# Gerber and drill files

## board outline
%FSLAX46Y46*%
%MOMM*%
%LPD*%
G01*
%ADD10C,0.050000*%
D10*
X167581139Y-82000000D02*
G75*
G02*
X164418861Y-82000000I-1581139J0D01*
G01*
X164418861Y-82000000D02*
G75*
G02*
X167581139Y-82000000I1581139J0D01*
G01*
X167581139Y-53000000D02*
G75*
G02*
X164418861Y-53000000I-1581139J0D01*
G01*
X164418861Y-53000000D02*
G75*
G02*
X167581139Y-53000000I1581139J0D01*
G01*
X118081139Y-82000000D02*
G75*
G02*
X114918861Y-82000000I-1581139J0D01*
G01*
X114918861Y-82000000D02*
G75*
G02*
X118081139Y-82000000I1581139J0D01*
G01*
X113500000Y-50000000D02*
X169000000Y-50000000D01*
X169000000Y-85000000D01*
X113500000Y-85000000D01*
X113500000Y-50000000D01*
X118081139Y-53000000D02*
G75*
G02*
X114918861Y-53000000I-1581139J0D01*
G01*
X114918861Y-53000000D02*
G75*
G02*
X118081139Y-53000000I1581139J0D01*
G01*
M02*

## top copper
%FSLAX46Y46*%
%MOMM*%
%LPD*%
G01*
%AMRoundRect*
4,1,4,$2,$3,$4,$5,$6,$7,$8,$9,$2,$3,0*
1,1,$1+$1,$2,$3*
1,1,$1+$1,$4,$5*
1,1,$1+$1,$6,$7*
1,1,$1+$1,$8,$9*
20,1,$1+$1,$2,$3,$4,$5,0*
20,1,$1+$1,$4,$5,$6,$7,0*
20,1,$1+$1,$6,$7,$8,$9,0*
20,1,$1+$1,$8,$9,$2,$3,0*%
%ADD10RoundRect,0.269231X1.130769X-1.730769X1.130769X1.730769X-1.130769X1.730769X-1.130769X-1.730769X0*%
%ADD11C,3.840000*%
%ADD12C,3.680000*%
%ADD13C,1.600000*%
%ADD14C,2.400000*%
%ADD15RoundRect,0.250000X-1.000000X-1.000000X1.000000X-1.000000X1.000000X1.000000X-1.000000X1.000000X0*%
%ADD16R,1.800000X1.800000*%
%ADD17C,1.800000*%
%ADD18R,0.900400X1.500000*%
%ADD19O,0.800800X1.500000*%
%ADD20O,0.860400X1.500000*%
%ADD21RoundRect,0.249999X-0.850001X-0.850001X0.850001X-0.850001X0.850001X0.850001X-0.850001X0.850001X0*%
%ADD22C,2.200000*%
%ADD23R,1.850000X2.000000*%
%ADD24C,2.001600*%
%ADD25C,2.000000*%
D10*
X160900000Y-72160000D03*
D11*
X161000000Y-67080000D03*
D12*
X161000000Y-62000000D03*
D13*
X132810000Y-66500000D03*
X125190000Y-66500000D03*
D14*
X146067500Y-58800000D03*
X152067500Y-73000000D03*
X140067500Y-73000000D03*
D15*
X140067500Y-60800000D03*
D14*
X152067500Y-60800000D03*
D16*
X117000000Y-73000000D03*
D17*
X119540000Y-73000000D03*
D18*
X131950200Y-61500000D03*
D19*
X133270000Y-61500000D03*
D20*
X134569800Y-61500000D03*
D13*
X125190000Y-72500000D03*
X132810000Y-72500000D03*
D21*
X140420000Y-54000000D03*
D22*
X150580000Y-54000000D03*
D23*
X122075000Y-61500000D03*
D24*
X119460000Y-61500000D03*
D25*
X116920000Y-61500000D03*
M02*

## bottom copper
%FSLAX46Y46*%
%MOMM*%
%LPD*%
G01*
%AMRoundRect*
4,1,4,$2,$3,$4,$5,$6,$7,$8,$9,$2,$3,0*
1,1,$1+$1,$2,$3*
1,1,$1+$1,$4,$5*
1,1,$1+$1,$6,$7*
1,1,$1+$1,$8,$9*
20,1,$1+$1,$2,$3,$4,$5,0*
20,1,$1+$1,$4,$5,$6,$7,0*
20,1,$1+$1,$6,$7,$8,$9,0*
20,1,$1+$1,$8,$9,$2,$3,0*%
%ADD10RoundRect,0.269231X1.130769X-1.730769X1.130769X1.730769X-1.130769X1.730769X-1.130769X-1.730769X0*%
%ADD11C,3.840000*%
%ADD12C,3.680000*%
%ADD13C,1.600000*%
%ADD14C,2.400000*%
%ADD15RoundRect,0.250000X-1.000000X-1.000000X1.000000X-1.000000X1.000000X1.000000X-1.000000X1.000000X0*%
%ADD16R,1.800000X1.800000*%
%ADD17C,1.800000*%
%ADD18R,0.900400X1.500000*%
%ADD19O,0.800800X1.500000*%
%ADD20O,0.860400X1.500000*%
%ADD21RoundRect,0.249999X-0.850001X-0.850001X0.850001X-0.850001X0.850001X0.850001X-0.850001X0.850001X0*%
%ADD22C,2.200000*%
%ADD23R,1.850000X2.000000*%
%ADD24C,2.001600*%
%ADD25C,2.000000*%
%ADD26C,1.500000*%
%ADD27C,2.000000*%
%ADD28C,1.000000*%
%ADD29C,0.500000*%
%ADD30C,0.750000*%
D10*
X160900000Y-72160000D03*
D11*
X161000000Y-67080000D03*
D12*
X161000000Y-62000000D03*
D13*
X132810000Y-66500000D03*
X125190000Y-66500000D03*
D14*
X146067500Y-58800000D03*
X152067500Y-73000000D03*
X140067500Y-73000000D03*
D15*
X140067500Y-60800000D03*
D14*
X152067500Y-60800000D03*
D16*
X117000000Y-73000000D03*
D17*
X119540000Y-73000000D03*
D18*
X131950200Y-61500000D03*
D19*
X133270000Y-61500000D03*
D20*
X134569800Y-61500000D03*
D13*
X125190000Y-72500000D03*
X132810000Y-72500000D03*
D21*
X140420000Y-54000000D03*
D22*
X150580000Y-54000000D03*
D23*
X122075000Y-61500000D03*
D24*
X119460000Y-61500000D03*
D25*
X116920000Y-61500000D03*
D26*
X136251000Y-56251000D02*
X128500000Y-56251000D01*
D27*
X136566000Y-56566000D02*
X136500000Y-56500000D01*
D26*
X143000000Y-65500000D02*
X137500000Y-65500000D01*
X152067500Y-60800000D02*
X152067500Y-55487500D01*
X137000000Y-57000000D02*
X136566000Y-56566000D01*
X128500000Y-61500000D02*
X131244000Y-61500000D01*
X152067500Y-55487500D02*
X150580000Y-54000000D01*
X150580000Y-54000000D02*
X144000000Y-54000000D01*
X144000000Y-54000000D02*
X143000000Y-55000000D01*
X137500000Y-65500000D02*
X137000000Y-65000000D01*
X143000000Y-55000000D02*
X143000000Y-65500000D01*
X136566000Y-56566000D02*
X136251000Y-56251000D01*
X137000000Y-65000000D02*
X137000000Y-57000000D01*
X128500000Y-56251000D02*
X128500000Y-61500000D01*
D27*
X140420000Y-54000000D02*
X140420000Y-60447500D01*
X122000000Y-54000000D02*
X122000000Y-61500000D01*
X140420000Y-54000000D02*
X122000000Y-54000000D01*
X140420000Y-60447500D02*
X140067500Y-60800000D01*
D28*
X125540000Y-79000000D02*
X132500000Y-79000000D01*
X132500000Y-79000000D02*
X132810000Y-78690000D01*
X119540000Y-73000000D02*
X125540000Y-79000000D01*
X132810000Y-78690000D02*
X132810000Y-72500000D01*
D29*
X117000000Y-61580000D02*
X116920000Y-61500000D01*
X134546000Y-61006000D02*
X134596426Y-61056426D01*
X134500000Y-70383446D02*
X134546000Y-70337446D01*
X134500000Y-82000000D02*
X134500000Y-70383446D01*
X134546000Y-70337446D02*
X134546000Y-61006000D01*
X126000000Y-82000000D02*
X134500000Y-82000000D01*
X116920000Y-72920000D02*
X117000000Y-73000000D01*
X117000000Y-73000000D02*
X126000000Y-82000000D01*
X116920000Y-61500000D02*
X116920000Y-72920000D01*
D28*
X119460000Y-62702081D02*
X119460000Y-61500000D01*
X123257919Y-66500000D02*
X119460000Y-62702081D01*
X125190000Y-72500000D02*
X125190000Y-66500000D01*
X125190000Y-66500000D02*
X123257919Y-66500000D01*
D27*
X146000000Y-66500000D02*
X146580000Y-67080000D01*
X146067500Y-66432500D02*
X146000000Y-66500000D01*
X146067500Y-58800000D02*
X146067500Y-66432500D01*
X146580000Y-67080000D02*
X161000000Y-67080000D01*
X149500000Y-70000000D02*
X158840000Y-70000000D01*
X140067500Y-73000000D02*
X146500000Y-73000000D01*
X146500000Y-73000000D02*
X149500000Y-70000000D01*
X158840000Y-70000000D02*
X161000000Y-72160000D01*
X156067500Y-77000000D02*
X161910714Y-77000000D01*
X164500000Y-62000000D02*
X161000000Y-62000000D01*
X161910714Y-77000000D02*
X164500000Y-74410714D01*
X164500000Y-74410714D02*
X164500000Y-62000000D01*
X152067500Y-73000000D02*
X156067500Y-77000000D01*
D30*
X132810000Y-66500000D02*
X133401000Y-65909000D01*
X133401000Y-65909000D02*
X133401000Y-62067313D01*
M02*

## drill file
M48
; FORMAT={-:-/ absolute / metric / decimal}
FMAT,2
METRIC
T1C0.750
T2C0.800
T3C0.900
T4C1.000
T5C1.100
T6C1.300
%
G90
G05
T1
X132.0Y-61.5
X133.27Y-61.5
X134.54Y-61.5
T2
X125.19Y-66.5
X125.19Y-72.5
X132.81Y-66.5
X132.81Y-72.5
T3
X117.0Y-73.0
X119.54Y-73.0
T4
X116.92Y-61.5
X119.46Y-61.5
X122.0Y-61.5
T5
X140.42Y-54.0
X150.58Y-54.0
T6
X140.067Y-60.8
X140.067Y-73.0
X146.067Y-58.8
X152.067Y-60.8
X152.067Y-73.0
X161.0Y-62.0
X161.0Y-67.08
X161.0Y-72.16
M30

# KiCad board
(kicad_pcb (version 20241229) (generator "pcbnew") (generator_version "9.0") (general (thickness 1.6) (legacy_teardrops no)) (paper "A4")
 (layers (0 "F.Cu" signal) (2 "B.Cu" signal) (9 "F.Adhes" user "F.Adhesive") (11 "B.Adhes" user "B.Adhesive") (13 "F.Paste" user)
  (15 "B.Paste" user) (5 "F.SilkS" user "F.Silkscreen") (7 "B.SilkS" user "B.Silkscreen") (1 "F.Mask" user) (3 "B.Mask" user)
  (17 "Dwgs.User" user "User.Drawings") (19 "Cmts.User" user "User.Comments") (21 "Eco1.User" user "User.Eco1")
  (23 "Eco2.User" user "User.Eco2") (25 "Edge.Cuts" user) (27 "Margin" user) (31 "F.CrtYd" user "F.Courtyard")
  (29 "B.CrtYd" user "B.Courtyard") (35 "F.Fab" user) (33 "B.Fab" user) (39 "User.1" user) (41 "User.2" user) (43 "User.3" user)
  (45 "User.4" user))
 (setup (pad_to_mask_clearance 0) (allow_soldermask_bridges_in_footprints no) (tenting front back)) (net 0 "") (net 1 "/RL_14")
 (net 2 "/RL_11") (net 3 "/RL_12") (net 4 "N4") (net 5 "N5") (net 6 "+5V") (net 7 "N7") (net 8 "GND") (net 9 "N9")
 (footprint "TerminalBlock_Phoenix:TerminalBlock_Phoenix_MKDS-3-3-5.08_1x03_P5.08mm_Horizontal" (layer "F.Cu") (at 161 72.16 90)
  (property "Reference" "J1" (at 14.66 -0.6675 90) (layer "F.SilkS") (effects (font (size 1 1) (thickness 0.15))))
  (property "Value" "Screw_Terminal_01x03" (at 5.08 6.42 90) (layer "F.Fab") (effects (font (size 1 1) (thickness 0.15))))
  (pad "1" thru_hole roundrect (at 0 0 90) (size 4 2.8) (drill 1.3 (offset 0 -0.1)) (layers "*.Cu" "*.Mask") (remove_unused_layers no)
   (roundrect_rratio 0.096154) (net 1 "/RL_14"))
  (pad "2" thru_hole circle (at 5.08 0 90) (size 3.84 3.84) (drill 1.3) (layers "*.Cu" "*.Mask") (remove_unused_layers no) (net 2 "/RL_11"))
  (pad "3" thru_hole circle (at 10.16 0 90) (size 3.68 3.68) (drill 1.3) (layers "*.Cu" "*.Mask") (remove_unused_layers no) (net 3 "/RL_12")))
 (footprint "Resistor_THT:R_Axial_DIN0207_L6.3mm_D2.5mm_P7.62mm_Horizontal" (layer "F.Cu") (at 132.81 66.5 180)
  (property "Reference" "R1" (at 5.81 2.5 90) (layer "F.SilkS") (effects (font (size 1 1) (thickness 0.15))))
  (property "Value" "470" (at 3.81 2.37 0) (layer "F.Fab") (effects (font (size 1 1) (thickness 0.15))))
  (pad "1" thru_hole circle (at 0 0 180) (size 1.6 1.6) (drill 0.8) (layers "*.Cu" "*.Mask") (remove_unused_layers no) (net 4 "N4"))
  (pad "2" thru_hole circle (at 7.62 0 180) (size 1.6 1.6) (drill 0.8) (layers "*.Cu" "*.Mask") (remove_unused_layers no) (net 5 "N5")))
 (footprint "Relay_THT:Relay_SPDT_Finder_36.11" (layer "F.Cu") (at 140.0675 60.8)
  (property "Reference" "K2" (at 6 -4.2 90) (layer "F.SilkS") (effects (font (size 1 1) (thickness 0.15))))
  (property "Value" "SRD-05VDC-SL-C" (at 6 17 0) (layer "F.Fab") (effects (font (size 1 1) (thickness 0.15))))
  (pad "11" thru_hole circle (at 6 -2) (size 2.4 2.4) (drill 1.3) (layers "*.Cu" "*.Mask") (remove_unused_layers no) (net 2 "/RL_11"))
  (pad "12" thru_hole circle (at 12 12.2) (size 2.4 2.4) (drill 1.3) (layers "*.Cu" "*.Mask") (remove_unused_layers no) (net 3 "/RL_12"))
  (pad "14" thru_hole circle (at 0 12.2) (size 2.4 2.4) (drill 1.3) (layers "*.Cu" "*.Mask") (remove_unused_layers no) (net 1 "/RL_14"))
  (pad "A1" thru_hole roundrect (at 0 0) (size 2.5 2.5) (drill 1.3) (layers "*.Cu" "*.Mask") (remove_unused_layers no)
   (roundrect_rratio 0.1) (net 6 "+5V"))
  (pad "A2" thru_hole circle (at 12 0) (size 2.4 2.4) (drill 1.3) (layers "*.Cu" "*.Mask") (remove_unused_layers no) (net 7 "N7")))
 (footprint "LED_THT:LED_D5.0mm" (layer "F.Cu") (at 117 73)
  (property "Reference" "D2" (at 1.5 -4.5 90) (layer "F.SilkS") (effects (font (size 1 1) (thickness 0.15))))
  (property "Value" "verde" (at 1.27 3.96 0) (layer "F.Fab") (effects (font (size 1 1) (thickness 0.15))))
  (pad "1" thru_hole rect (at 0 0) (size 1.8 1.8) (drill 0.9) (layers "*.Cu" "*.Mask") (remove_unused_layers no) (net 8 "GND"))
  (pad "2" thru_hole circle (at 2.54 0) (size 1.8 1.8) (drill 0.9) (layers "*.Cu" "*.Mask") (remove_unused_layers no) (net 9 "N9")))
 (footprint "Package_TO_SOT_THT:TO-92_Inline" (layer "F.Cu") (at 132 61.5)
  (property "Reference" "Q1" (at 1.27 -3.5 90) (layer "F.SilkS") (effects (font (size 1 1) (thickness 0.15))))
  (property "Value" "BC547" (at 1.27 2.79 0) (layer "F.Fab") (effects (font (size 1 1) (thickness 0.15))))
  (pad "1" thru_hole rect (at 0 0) (size 0.9004 1.5) (drill 0.75 (offset -0.0498 0)) (layers "*.Cu" "*.Mask") (remove_unused_layers no)
   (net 7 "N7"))
  (pad "2" thru_hole oval (at 1.27 0) (size 0.8008 1.5) (drill 0.75) (layers "*.Cu" "*.Mask") (remove_unused_layers no) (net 4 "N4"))
  (pad "3" thru_hole oval (at 2.54 0) (size 0.8604 1.5) (drill 0.75 (offset 0.0298 0)) (layers "*.Cu" "*.Mask") (remove_unused_layers no)
   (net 8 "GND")))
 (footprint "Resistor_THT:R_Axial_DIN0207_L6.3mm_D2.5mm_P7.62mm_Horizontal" (layer "F.Cu") (at 125.19 72.5)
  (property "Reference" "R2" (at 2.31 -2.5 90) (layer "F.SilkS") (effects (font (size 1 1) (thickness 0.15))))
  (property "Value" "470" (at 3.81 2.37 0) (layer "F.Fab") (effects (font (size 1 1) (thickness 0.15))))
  (pad "1" thru_hole circle (at 0 0) (size 1.6 1.6) (drill 0.8) (layers "*.Cu" "*.Mask") (remove_unused_layers no) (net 5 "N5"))
  (pad "2" thru_hole circle (at 7.62 0) (size 1.6 1.6) (drill 0.8) (layers "*.Cu" "*.Mask") (remove_unused_layers no) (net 9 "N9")))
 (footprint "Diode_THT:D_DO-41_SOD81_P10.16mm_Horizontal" (layer "F.Cu") (at 140.42 54)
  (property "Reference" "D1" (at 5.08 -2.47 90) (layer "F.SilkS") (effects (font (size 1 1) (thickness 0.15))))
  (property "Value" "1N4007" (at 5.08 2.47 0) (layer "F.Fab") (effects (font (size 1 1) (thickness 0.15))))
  (pad "1" thru_hole roundrect (at 0 0) (size 2.2 2.2) (drill 1.1) (layers "*.Cu" "*.Mask") (remove_unused_layers no)
   (roundrect_rratio 0.113636) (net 6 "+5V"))
  (pad "2" thru_hole circle (at 10.16 0) (size 2.2 2.2) (drill 1.1) (layers "*.Cu" "*.Mask") (remove_unused_layers no) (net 7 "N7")))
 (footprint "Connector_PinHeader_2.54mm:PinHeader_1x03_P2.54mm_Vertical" (layer "F.Cu") (at 122 61.5 -90)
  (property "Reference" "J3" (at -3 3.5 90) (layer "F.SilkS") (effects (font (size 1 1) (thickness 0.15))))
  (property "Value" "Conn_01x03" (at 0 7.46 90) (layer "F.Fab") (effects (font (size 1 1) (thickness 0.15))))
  (pad "1" thru_hole rect (at 0 0 270) (size 2 1.85) (drill 1 (offset 0 -0.075)) (layers "*.Cu" "*.Mask") (remove_unused_layers no)
   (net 6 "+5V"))
  (pad "2" thru_hole circle (at 0 2.54 270) (size 2.0016 2.0016) (drill 1) (layers "*.Cu" "*.Mask") (remove_unused_layers no) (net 5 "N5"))
  (pad "3" thru_hole circle (at 0 5.08 270) (size 2 2) (drill 1) (layers "*.Cu" "*.Mask") (remove_unused_layers no) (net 8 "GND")))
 (gr_circle (center 166 82) (end 166.5 83.5) (stroke (width 0.05) (type default)) (fill no) (layer "Edge.Cuts"))
 (gr_circle (center 166 53) (end 166.5 54.5) (stroke (width 0.05) (type default)) (fill no) (layer "Edge.Cuts"))
 (gr_circle (center 116.5 82) (end 117 83.5) (stroke (width 0.05) (type default)) (fill no) (layer "Edge.Cuts"))
 (gr_rect (start 113.5 50) (end 169 85) (stroke (width 0.05) (type default)) (fill no) (layer "Edge.Cuts"))
 (gr_circle (center 116.5 53) (end 117 54.5) (stroke (width 0.05) (type default)) (fill no) (layer "Edge.Cuts"))
 (segment (start 136.251 56.251) (end 128.5 56.251) (width 1.5) (layer "B.Cu") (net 7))
 (segment (start 136.566 56.566) (end 136.5 56.5) (width 2) (layer "B.Cu") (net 7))
 (segment (start 143 65.5) (end 137.5 65.5) (width 1.5) (layer "B.Cu") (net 7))
 (segment (start 152.0675 60.8) (end 152.0675 55.4875) (width 1.5) (layer "B.Cu") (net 7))
 (segment (start 137 57) (end 136.566 56.566) (width 1.5) (layer "B.Cu") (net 7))
 (segment (start 128.5 61.5) (end 131.244 61.5) (width 1.5) (layer "B.Cu") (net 7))
 (segment (start 152.0675 55.4875) (end 150.58 54) (width 1.5) (layer "B.Cu") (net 7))
 (segment (start 150.58 54) (end 144 54) (width 1.5) (layer "B.Cu") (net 7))
 (segment (start 144 54) (end 143 55) (width 1.5) (layer "B.Cu") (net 7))
 (segment (start 137.5 65.5) (end 137 65) (width 1.5) (layer "B.Cu") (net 7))
 (segment (start 143 55) (end 143 65.5) (width 1.5) (layer "B.Cu") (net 7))
 (segment (start 136.566 56.566) (end 136.251 56.251) (width 1.5) (layer "B.Cu") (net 7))
 (segment (start 137 65) (end 137 57) (width 1.5) (layer "B.Cu") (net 7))
 (segment (start 128.5 56.251) (end 128.5 61.5) (width 1.5) (layer "B.Cu") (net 7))
 (segment (start 140.42 54) (end 140.42 60.4475) (width 2) (layer "B.Cu") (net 6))
 (segment (start 122 54) (end 122 61.5) (width 2) (layer "B.Cu") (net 6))
 (segment (start 140.42 54) (end 122 54) (width 2) (layer "B.Cu") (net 6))
 (segment (start 140.42 60.4475) (end 140.0675 60.8) (width 2) (layer "B.Cu") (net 6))
 (segment (start 125.54 79) (end 132.5 79) (width 1) (layer "B.Cu") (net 9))
 (segment (start 132.5 79) (end 132.81 78.69) (width 1) (layer "B.Cu") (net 9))
 (segment (start 119.54 73) (end 125.54 79) (width 1) (layer "B.Cu") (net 9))
 (segment (start 132.81 78.69) (end 132.81 72.5) (width 1) (layer "B.Cu") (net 9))
 (segment (start 117 61.58) (end 116.92 61.5) (width 0.5) (layer "B.Cu") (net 8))
 (segment (start 134.546 61.006) (end 134.596426 61.056426) (width 0.5) (layer "B.Cu") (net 8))
 (segment (start 134.5 70.383446) (end 134.546 70.337446) (width 0.5) (layer "B.Cu") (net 8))
 (segment (start 134.5 82) (end 134.5 70.383446) (width 0.5) (layer "B.Cu") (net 8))
 (segment (start 134.546 70.337446) (end 134.546 61.006) (width 0.5) (layer "B.Cu") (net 8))
 (segment (start 126 82) (end 134.5 82) (width 0.5) (layer "B.Cu") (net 8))
 (segment (start 116.92 72.92) (end 117 73) (width 0.5) (layer "B.Cu") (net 8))
 (segment (start 117 73) (end 126 82) (width 0.5) (layer "B.Cu") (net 8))
 (segment (start 116.92 61.5) (end 116.92 72.92) (width 0.5) (layer "B.Cu") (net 8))
 (segment (start 119.46 62.702081) (end 119.46 61.5) (width 1) (layer "B.Cu") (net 5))
 (segment (start 123.257919 66.5) (end 119.46 62.702081) (width 1) (layer "B.Cu") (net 5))
 (segment (start 125.19 72.5) (end 125.19 66.5) (width 1) (layer "B.Cu") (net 5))
 (segment (start 125.19 66.5) (end 123.257919 66.5) (width 1) (layer "B.Cu") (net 5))
 (segment (start 146 66.5) (end 146.58 67.08) (width 2) (layer "B.Cu") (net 2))
 (segment (start 146.0675 66.4325) (end 146 66.5) (width 2) (layer "B.Cu") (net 2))
 (segment (start 146.0675 58.8) (end 146.0675 66.4325) (width 2) (layer "B.Cu") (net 2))
 (segment (start 146.58 67.08) (end 161 67.08) (width 2) (layer "B.Cu") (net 2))
 (segment (start 149.5 70) (end 158.84 70) (width 2) (layer "B.Cu") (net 1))
 (segment (start 140.0675 73) (end 146.5 73) (width 2) (layer "B.Cu") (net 1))
 (segment (start 146.5 73) (end 149.5 70) (width 2) (layer "B.Cu") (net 1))
 (segment (start 158.84 70) (end 161 72.16) (width 2) (layer "B.Cu") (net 1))
 (segment (start 156.0675 77) (end 161.910714 77) (width 2) (layer "B.Cu") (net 3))
 (segment (start 164.5 62) (end 161 62) (width 2) (layer "B.Cu") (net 3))
 (segment (start 161.910714 77) (end 164.5 74.410714) (width 2) (layer "B.Cu") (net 3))
 (segment (start 164.5 74.410714) (end 164.5 62) (width 2) (layer "B.Cu") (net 3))
 (segment (start 152.0675 73) (end 156.0675 77) (width 2) (layer "B.Cu") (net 3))
 (segment (start 132.81 66.5) (end 133.401 65.909) (width 0.75) (layer "B.Cu") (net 4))
 (segment (start 133.401 65.909) (end 133.401 62.067313) (width 0.75) (layer "B.Cu") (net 4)))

